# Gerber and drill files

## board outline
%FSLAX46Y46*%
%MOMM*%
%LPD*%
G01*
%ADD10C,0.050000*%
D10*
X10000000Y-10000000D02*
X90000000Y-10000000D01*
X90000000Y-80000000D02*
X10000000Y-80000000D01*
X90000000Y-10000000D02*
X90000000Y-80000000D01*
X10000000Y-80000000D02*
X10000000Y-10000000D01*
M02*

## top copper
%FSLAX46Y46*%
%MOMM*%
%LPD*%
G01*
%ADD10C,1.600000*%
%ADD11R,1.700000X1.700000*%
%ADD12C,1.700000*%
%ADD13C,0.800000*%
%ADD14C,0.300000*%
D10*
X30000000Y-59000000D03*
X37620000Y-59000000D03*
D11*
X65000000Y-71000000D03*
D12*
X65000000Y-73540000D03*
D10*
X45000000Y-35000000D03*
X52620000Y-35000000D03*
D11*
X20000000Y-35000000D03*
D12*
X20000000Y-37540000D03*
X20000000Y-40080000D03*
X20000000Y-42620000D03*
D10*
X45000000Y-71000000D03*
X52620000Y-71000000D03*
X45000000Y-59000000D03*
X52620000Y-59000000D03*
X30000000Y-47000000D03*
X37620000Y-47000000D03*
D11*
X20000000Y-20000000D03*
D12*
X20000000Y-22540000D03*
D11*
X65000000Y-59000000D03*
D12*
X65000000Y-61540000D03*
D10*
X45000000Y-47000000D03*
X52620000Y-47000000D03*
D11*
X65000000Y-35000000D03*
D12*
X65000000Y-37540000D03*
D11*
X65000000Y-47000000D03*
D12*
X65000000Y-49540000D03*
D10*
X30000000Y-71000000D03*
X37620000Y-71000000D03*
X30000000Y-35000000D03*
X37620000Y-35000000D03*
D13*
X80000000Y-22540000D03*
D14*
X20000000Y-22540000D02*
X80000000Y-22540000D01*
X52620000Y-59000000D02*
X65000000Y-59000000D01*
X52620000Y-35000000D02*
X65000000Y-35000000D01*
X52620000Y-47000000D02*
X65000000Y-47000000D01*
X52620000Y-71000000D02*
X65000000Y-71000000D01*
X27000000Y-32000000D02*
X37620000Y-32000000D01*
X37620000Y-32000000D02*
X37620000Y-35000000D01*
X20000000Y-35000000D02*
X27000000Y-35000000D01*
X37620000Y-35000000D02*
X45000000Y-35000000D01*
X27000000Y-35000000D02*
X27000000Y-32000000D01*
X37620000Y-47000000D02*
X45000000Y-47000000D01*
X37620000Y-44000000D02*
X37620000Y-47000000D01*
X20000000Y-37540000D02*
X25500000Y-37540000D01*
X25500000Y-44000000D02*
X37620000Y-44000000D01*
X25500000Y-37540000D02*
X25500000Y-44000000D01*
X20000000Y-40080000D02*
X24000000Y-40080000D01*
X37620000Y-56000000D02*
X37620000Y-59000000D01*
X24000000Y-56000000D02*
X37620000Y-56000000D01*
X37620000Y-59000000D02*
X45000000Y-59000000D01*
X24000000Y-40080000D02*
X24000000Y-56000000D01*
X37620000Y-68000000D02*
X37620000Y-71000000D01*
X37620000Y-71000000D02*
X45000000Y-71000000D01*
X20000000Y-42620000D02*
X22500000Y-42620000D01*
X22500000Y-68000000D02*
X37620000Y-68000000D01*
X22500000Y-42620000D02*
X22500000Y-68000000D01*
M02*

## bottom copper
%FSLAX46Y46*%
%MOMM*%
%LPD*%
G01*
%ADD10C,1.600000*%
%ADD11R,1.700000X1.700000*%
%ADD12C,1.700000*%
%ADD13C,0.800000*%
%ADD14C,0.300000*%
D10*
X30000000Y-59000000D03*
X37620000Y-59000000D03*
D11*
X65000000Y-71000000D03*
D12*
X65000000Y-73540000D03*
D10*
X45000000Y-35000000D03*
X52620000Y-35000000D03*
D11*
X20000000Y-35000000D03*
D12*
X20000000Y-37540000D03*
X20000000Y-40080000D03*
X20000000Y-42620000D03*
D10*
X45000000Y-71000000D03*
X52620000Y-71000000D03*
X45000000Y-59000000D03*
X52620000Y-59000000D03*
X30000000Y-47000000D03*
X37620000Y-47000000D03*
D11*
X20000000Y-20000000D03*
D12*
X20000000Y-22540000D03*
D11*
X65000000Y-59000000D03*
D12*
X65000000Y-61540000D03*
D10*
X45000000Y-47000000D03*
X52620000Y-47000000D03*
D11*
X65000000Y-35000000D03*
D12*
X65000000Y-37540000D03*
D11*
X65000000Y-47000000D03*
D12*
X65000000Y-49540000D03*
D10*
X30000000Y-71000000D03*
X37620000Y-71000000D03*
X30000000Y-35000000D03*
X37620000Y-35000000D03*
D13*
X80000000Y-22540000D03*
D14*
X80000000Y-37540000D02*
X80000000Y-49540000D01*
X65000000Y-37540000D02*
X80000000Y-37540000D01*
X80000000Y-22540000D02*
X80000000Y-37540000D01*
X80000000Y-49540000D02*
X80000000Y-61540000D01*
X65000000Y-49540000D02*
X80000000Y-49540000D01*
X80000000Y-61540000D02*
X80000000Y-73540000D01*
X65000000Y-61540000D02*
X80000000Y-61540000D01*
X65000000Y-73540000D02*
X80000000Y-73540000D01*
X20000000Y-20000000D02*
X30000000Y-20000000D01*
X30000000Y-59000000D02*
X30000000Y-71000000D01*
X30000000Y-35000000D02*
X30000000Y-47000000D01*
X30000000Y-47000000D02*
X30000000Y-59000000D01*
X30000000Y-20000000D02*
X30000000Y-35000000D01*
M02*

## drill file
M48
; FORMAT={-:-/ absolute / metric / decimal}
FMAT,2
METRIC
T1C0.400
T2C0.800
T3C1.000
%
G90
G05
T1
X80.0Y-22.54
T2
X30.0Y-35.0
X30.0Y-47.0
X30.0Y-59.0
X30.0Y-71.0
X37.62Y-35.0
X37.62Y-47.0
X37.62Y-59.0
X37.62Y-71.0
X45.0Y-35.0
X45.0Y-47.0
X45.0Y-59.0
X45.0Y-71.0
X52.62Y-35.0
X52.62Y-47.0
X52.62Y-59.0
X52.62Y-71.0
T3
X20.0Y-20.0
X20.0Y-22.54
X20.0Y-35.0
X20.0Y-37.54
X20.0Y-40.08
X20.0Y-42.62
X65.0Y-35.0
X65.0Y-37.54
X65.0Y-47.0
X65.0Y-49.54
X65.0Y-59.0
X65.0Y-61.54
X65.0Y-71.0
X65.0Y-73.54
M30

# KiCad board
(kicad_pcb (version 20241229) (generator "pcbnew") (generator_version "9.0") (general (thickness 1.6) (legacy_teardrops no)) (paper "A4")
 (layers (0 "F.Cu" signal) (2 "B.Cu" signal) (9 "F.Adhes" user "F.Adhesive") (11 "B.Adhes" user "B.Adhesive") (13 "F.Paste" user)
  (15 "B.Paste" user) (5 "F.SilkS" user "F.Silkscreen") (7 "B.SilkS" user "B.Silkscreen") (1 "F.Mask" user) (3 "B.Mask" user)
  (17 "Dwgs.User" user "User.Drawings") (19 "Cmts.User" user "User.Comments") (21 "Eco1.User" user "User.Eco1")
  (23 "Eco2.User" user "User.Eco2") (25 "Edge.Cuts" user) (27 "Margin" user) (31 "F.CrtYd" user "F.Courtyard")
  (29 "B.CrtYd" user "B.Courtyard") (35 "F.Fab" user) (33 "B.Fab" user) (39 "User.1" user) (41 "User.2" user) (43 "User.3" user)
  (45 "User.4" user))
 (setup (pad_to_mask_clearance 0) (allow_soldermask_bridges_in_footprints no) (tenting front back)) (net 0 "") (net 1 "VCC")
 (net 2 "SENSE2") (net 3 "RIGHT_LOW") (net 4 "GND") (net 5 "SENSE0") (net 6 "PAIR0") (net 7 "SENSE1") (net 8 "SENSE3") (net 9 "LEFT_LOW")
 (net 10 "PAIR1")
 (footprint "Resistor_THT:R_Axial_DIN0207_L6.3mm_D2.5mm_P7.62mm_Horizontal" (layer "F.Cu") (at 30 59)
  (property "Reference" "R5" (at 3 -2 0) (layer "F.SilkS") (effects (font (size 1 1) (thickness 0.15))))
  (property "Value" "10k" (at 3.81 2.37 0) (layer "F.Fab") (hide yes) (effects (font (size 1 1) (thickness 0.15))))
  (pad "1" thru_hole circle (at 0 0) (size 1.6 1.6) (drill 0.8) (layers "*.Cu" "*.Mask") (remove_unused_layers no) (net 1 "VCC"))
  (pad "2" thru_hole circle (at 7.62 0) (size 1.6 1.6) (drill 0.8) (layers "*.Cu" "*.Mask") (remove_unused_layers no) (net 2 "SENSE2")))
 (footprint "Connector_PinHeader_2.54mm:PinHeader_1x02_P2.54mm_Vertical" (layer "F.Cu") (at 65 71)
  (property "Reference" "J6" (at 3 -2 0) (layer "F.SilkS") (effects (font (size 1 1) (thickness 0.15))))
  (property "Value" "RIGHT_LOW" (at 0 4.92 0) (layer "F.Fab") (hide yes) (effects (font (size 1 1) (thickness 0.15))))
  (pad "1" thru_hole rect (at 0 0) (size 1.7 1.7) (drill 1) (layers "*.Cu" "*.Mask") (remove_unused_layers no) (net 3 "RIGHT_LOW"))
  (pad "2" thru_hole circle (at 0 2.54) (size 1.7 1.7) (drill 1) (layers "*.Cu" "*.Mask") (remove_unused_layers no) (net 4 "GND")))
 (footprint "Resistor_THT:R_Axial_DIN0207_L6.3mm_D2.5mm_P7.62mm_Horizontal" (layer "F.Cu") (at 45 35)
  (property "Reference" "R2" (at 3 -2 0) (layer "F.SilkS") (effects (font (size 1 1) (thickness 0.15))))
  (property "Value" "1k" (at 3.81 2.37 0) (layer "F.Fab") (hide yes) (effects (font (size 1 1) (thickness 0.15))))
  (pad "1" thru_hole circle (at 0 0) (size 1.6 1.6) (drill 0.8) (layers "*.Cu" "*.Mask") (remove_unused_layers no) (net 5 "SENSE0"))
  (pad "2" thru_hole circle (at 7.62 0) (size 1.6 1.6) (drill 0.8) (layers "*.Cu" "*.Mask") (remove_unused_layers no) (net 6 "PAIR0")))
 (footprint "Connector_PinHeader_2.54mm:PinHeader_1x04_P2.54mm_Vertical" (layer "F.Cu") (at 20 35)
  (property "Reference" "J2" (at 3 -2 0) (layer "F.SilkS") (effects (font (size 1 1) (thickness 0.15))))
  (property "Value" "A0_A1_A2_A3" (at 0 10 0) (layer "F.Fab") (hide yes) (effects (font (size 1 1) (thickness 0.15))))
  (pad "1" thru_hole rect (at 0 0) (size 1.7 1.7) (drill 1) (layers "*.Cu" "*.Mask") (remove_unused_layers no) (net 5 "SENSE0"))
  (pad "2" thru_hole circle (at 0 2.54) (size 1.7 1.7) (drill 1) (layers "*.Cu" "*.Mask") (remove_unused_layers no) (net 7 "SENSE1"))
  (pad "3" thru_hole circle (at 0 5.08) (size 1.7 1.7) (drill 1) (layers "*.Cu" "*.Mask") (remove_unused_layers no) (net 2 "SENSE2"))
  (pad "4" thru_hole circle (at 0 7.62) (size 1.7 1.7) (drill 1) (layers "*.Cu" "*.Mask") (remove_unused_layers no) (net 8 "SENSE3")))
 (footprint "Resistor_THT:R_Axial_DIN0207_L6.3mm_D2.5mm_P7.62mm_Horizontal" (layer "F.Cu") (at 45 71)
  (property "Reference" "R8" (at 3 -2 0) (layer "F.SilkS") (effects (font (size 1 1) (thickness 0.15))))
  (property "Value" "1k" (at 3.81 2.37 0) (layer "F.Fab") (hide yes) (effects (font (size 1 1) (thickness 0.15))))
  (pad "1" thru_hole circle (at 0 0) (size 1.6 1.6) (drill 0.8) (layers "*.Cu" "*.Mask") (remove_unused_layers no) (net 8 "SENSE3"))
  (pad "2" thru_hole circle (at 7.62 0) (size 1.6 1.6) (drill 0.8) (layers "*.Cu" "*.Mask") (remove_unused_layers no) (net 3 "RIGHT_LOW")))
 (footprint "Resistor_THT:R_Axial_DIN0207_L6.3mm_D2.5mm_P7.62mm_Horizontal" (layer "F.Cu") (at 45 59)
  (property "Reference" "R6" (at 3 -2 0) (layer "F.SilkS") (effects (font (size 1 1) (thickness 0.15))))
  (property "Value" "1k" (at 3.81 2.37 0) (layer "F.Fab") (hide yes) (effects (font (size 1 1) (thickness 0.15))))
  (pad "1" thru_hole circle (at 0 0) (size 1.6 1.6) (drill 0.8) (layers "*.Cu" "*.Mask") (remove_unused_layers no) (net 2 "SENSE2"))
  (pad "2" thru_hole circle (at 7.62 0) (size 1.6 1.6) (drill 0.8) (layers "*.Cu" "*.Mask") (remove_unused_layers no) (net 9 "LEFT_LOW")))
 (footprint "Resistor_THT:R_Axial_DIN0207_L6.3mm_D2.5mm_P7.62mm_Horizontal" (layer "F.Cu") (at 30 47)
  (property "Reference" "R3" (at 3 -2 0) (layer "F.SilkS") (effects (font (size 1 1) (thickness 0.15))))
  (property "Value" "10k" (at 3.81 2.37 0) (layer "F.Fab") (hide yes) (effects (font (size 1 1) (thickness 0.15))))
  (pad "1" thru_hole circle (at 0 0) (size 1.6 1.6) (drill 0.8) (layers "*.Cu" "*.Mask") (remove_unused_layers no) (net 1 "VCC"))
  (pad "2" thru_hole circle (at 7.62 0) (size 1.6 1.6) (drill 0.8) (layers "*.Cu" "*.Mask") (remove_unused_layers no) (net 7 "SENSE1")))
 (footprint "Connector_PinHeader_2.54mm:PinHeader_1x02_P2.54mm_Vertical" (layer "F.Cu") (at 20 20)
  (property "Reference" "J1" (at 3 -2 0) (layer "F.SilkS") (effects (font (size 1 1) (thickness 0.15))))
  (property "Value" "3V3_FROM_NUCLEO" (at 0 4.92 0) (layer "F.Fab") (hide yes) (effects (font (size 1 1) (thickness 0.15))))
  (pad "1" thru_hole rect (at 0 0) (size 1.7 1.7) (drill 1) (layers "*.Cu" "*.Mask") (remove_unused_layers no) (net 1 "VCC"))
  (pad "2" thru_hole circle (at 0 2.54) (size 1.7 1.7) (drill 1) (layers "*.Cu" "*.Mask") (remove_unused_layers no) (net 4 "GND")))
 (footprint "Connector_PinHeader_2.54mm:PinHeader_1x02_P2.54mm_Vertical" (layer "F.Cu") (at 65 59)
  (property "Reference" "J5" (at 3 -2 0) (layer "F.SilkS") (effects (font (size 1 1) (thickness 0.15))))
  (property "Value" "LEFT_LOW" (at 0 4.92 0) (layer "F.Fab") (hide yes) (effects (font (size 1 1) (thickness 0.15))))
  (pad "1" thru_hole rect (at 0 0) (size 1.7 1.7) (drill 1) (layers "*.Cu" "*.Mask") (remove_unused_layers no) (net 9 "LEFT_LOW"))
  (pad "2" thru_hole circle (at 0 2.54) (size 1.7 1.7) (drill 1) (layers "*.Cu" "*.Mask") (remove_unused_layers no) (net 4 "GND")))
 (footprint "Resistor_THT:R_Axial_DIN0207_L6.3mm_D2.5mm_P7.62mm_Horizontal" (layer "F.Cu") (at 45 47)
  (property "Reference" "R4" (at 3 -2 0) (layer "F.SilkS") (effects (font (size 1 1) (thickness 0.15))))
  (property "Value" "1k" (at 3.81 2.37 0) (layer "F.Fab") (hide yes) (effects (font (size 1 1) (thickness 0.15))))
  (pad "1" thru_hole circle (at 0 0) (size 1.6 1.6) (drill 0.8) (layers "*.Cu" "*.Mask") (remove_unused_layers no) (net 7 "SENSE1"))
  (pad "2" thru_hole circle (at 7.62 0) (size 1.6 1.6) (drill 0.8) (layers "*.Cu" "*.Mask") (remove_unused_layers no) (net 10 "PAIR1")))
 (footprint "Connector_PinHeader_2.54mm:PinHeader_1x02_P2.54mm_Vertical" (layer "F.Cu") (at 65 35)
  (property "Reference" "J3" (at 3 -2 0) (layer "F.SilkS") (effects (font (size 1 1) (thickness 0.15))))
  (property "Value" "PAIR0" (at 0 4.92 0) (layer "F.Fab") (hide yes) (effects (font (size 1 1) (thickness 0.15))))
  (pad "1" thru_hole rect (at 0 0) (size 1.7 1.7) (drill 1) (layers "*.Cu" "*.Mask") (remove_unused_layers no) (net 6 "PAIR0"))
  (pad "2" thru_hole circle (at 0 2.54) (size 1.7 1.7) (drill 1) (layers "*.Cu" "*.Mask") (remove_unused_layers no) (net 4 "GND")))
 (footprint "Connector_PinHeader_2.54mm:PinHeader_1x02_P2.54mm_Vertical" (layer "F.Cu") (at 65 47)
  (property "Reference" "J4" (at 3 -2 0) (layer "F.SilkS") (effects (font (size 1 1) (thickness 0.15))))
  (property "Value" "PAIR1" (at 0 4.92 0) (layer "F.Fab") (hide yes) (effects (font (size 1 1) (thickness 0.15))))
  (pad "1" thru_hole rect (at 0 0) (size 1.7 1.7) (drill 1) (layers "*.Cu" "*.Mask") (remove_unused_layers no) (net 10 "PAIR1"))
  (pad "2" thru_hole circle (at 0 2.54) (size 1.7 1.7) (drill 1) (layers "*.Cu" "*.Mask") (remove_unused_layers no) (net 4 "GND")))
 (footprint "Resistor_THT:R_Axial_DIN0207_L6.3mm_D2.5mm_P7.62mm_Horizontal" (layer "F.Cu") (at 30 71)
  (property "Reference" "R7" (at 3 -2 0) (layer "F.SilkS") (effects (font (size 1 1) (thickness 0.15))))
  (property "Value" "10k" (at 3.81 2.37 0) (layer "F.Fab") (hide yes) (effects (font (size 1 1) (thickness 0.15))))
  (pad "1" thru_hole circle (at 0 0) (size 1.6 1.6) (drill 0.8) (layers "*.Cu" "*.Mask") (remove_unused_layers no) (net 1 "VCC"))
  (pad "2" thru_hole circle (at 7.62 0) (size 1.6 1.6) (drill 0.8) (layers "*.Cu" "*.Mask") (remove_unused_layers no) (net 8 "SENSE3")))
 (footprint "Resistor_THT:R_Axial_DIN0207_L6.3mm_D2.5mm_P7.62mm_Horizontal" (layer "F.Cu") (at 30 35)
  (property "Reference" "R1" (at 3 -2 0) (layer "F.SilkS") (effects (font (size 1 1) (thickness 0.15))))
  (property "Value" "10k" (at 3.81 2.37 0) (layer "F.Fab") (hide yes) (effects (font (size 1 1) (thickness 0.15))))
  (pad "1" thru_hole circle (at 0 0) (size 1.6 1.6) (drill 0.8) (layers "*.Cu" "*.Mask") (remove_unused_layers no) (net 1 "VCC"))
  (pad "2" thru_hole circle (at 7.62 0) (size 1.6 1.6) (drill 0.8) (layers "*.Cu" "*.Mask") (remove_unused_layers no) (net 5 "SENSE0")))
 (gr_line (start 10 10) (end 90 10) (stroke (width 0.05) (type default)) (layer "Edge.Cuts"))
 (gr_line (start 90 80) (end 10 80) (stroke (width 0.05) (type default)) (layer "Edge.Cuts"))
 (gr_line (start 90 10) (end 90 80) (stroke (width 0.05) (type default)) (layer "Edge.Cuts"))
 (gr_line (start 10 80) (end 10 10) (stroke (width 0.05) (type default)) (layer "Edge.Cuts"))
 (segment (start 20 22.54) (end 80 22.54) (width 0.3) (layer "F.Cu") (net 4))
 (via (at 80 22.54) (size 0.8) (drill 0.4) (layers "F.Cu" "B.Cu") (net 4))
 (segment (start 80 37.54) (end 80 49.54) (width 0.3) (layer "B.Cu") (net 4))
 (segment (start 65 37.54) (end 80 37.54) (width 0.3) (layer "B.Cu") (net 4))
 (segment (start 80 22.54) (end 80 37.54) (width 0.3) (layer "B.Cu") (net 4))
 (segment (start 80 49.54) (end 80 61.54) (width 0.3) (layer "B.Cu") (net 4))
 (segment (start 65 49.54) (end 80 49.54) (width 0.3) (layer "B.Cu") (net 4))
 (segment (start 80 61.54) (end 80 73.54) (width 0.3) (layer "B.Cu") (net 4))
 (segment (start 65 61.54) (end 80 61.54) (width 0.3) (layer "B.Cu") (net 4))
 (segment (start 65 73.54) (end 80 73.54) (width 0.3) (layer "B.Cu") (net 4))
 (segment (start 52.62 59) (end 65 59) (width 0.3) (layer "F.Cu") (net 9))
 (segment (start 52.62 35) (end 65 35) (width 0.3) (layer "F.Cu") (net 6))
 (segment (start 52.62 47) (end 65 47) (width 0.3) (layer "F.Cu") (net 10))
 (segment (start 52.62 71) (end 65 71) (width 0.3) (layer "F.Cu") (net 3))
 (segment (start 27 32) (end 37.62 32) (width 0.3) (layer "F.Cu") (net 5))
 (segment (start 37.62 32) (end 37.62 35) (width 0.3) (layer "F.Cu") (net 5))
 (segment (start 20 35) (end 27 35) (width 0.3) (layer "F.Cu") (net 5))
 (segment (start 37.62 35) (end 45 35) (width 0.3) (layer "F.Cu") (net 5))
 (segment (start 27 35) (end 27 32) (width 0.3) (layer "F.Cu") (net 5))
 (segment (start 37.62 47) (end 45 47) (width 0.3) (layer "F.Cu") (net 7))
 (segment (start 37.62 44) (end 37.62 47) (width 0.3) (layer "F.Cu") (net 7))
 (segment (start 20 37.54) (end 25.5 37.54) (width 0.3) (layer "F.Cu") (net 7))
 (segment (start 25.5 44) (end 37.62 44) (width 0.3) (layer "F.Cu") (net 7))
 (segment (start 25.5 37.54) (end 25.5 44) (width 0.3) (layer "F.Cu") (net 7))
 (segment (start 20 40.08) (end 24 40.08) (width 0.3) (layer "F.Cu") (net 2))
 (segment (start 37.62 56) (end 37.62 59) (width 0.3) (layer "F.Cu") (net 2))
 (segment (start 24 56) (end 37.62 56) (width 0.3) (layer "F.Cu") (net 2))
 (segment (start 37.62 59) (end 45 59) (width 0.3) (layer "F.Cu") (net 2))
 (segment (start 24 40.08) (end 24 56) (width 0.3) (layer "F.Cu") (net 2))
 (segment (start 37.62 68) (end 37.62 71) (width 0.3) (layer "F.Cu") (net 8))
 (segment (start 37.62 71) (end 45 71) (width 0.3) (layer "F.Cu") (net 8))
 (segment (start 20 42.62) (end 22.5 42.62) (width 0.3) (layer "F.Cu") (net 8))
 (segment (start 22.5 68) (end 37.62 68) (width 0.3) (layer "F.Cu") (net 8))
 (segment (start 22.5 42.62) (end 22.5 68) (width 0.3) (layer "F.Cu") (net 8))
 (segment (start 20 20) (end 30 20) (width 0.3) (layer "B.Cu") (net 1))
 (segment (start 30 59) (end 30 71) (width 0.3) (layer "B.Cu") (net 1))
 (segment (start 30 35) (end 30 47) (width 0.3) (layer "B.Cu") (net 1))
 (segment (start 30 47) (end 30 59) (width 0.3) (layer "B.Cu") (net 1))
 (segment (start 30 20) (end 30 35) (width 0.3) (layer "B.Cu") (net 1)))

